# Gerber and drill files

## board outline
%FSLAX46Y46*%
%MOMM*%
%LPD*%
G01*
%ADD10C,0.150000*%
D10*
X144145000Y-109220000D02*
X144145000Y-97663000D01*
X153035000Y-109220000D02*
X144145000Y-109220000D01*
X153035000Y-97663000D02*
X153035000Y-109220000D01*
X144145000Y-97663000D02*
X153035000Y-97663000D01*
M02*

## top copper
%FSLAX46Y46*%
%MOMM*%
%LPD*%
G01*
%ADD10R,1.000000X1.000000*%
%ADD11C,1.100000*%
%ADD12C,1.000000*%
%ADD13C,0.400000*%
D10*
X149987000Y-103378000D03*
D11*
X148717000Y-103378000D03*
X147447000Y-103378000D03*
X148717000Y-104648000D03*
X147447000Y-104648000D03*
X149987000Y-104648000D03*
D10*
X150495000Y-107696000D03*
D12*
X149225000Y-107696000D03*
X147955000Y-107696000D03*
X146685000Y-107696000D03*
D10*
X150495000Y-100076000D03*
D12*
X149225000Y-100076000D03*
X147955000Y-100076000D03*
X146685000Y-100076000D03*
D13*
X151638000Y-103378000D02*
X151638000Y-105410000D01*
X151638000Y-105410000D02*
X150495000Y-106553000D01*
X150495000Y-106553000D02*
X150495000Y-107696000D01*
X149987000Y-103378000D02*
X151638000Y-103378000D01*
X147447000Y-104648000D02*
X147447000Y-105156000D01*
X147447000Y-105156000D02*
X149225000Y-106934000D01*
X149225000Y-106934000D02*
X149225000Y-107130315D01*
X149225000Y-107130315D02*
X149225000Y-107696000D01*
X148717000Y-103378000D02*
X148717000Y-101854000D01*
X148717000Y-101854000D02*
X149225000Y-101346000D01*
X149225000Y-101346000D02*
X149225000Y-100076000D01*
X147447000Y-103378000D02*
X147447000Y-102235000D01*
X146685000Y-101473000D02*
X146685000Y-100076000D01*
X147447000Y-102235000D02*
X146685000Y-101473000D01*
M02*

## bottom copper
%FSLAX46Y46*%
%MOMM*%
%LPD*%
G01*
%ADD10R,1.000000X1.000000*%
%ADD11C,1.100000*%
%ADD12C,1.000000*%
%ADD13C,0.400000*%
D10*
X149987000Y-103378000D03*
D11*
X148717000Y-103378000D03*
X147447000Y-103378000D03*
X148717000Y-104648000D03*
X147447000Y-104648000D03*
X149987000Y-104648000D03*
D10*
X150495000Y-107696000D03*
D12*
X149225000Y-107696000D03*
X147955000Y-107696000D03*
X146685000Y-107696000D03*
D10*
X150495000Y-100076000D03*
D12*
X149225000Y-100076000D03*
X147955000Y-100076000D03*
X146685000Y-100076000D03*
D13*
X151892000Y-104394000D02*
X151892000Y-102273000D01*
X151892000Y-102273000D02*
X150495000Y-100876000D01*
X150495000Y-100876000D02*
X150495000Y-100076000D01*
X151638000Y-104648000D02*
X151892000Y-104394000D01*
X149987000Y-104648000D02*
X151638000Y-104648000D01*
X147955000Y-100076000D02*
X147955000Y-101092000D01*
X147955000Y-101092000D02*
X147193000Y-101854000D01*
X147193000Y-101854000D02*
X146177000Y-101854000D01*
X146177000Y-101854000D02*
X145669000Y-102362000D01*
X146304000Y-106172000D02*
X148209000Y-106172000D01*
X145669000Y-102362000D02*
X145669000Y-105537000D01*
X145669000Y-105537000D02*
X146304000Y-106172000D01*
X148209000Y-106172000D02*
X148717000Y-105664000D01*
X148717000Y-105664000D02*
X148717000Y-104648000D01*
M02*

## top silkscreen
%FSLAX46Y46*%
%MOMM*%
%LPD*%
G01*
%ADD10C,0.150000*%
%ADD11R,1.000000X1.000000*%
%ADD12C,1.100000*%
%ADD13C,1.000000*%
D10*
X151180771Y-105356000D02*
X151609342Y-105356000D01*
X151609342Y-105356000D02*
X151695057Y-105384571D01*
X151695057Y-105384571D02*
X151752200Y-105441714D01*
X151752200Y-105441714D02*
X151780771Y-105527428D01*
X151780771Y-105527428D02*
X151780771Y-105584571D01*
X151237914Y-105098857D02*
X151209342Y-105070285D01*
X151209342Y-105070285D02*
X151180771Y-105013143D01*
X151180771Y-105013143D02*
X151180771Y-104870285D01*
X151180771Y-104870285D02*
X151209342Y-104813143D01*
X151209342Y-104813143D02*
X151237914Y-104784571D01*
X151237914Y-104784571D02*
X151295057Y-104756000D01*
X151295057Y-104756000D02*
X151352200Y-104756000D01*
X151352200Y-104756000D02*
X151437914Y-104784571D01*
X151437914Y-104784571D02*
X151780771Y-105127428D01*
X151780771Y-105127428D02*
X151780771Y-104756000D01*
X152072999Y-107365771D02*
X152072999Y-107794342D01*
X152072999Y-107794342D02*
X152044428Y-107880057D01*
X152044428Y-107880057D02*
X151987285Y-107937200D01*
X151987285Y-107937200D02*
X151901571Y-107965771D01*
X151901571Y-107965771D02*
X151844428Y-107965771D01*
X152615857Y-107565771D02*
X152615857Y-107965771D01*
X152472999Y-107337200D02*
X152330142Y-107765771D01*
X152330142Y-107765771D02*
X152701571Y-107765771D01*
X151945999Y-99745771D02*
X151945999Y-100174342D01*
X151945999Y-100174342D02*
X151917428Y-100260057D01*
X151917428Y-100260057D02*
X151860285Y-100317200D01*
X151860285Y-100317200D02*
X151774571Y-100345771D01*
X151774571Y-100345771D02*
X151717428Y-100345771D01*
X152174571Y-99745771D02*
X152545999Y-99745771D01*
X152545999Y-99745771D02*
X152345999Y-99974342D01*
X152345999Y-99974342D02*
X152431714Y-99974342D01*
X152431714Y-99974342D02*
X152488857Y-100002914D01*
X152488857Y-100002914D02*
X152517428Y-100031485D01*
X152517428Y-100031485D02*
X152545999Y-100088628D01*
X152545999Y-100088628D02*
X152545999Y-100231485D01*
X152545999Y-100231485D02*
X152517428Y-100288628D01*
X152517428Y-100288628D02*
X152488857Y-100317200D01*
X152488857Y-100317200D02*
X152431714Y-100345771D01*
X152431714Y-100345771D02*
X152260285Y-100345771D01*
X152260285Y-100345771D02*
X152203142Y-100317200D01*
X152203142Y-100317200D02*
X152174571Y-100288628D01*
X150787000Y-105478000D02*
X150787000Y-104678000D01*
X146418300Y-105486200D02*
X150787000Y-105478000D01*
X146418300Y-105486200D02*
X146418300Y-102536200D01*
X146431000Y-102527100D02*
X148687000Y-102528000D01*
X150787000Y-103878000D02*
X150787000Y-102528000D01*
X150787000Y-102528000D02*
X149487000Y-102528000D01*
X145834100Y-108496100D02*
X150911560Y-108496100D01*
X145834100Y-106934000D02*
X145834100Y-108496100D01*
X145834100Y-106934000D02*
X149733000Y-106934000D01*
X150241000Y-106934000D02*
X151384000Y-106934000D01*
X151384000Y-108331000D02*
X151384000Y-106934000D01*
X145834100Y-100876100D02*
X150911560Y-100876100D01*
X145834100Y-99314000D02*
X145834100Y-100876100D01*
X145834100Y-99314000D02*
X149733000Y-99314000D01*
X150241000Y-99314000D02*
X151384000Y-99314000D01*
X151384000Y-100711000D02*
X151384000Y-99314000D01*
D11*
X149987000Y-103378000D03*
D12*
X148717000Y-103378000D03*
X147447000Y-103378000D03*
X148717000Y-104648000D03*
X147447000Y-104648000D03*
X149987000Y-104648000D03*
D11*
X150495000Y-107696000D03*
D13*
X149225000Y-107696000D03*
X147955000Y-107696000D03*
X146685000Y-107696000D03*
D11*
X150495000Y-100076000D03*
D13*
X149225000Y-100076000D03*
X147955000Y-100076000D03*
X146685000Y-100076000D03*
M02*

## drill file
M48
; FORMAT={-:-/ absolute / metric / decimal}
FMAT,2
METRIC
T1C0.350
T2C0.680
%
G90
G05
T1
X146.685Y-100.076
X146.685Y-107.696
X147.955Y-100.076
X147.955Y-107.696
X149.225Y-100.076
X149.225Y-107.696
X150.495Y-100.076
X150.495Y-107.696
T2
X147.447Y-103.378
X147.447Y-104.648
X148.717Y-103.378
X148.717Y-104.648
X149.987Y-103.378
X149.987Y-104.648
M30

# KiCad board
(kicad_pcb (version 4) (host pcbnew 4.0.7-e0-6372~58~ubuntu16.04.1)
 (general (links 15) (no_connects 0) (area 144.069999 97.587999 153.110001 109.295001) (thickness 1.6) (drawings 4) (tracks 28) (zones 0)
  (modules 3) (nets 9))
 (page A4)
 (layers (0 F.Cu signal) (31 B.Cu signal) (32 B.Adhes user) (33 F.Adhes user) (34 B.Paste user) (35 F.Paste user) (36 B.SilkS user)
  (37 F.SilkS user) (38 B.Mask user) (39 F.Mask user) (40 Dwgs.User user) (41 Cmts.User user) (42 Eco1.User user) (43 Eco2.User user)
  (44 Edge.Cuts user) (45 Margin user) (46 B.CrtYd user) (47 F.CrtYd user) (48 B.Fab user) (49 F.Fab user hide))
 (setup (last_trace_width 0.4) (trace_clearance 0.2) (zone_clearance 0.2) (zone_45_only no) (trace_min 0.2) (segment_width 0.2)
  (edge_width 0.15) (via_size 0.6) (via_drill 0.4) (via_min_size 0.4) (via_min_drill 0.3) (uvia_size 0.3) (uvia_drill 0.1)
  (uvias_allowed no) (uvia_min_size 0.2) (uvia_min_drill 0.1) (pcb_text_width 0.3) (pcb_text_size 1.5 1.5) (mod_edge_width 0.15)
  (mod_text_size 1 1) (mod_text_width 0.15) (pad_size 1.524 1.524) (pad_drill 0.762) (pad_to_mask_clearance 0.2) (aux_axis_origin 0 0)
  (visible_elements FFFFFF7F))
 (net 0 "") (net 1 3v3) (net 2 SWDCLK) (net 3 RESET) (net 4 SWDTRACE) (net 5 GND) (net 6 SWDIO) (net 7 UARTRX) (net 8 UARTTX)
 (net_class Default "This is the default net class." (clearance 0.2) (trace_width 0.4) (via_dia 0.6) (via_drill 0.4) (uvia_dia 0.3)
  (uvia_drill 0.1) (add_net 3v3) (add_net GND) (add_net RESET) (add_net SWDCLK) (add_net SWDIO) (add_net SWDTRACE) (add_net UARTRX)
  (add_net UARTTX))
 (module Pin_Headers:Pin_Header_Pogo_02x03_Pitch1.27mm (layer F.Cu) (at 149.987 103.378 270)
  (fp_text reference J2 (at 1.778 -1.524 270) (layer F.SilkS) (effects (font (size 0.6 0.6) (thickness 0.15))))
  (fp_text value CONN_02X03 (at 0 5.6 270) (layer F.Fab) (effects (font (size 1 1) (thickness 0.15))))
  (fp_line (start 2.1 -0.8) (end 1.3 -0.8) (layer F.SilkS) (width 0.15))
  (fp_line (start 2.1082 3.5687) (end 2.1 -0.8) (layer F.SilkS) (width 0.15))
  (fp_line (start 2.1082 3.5687) (end -0.8418 3.5687) (layer F.SilkS) (width 0.15))
  (fp_line (start -0.8509 3.556) (end -0.85 1.3) (layer F.SilkS) (width 0.15))
  (fp_line (start 0.5 -0.8) (end -0.85 -0.8) (layer F.SilkS) (width 0.15))
  (fp_line (start -0.85 -0.8) (end -0.85 0.5) (layer F.SilkS) (width 0.15))
  (pad 1 thru_hole rect (at 0 0 270) (size 1 1) (drill 0.68) (layers *.Cu *.Mask F.SilkS) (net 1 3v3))
  (pad 3 thru_hole circle (at 0 1.27 270) (size 1.1 1.1) (drill 0.68) (layers *.Cu *.Mask F.SilkS) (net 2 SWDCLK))
  (pad 5 thru_hole circle (at 0 2.54 270) (size 1.1 1.1) (drill 0.68) (layers *.Cu *.Mask F.SilkS) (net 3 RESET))
  (pad 4 thru_hole circle (at 1.27 1.27 270) (size 1.1 1.1) (drill 0.68) (layers *.Cu *.Mask F.SilkS) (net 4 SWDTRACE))
  (pad 6 thru_hole circle (at 1.27 2.54 270) (size 1.1 1.1) (drill 0.68) (layers *.Cu *.Mask F.SilkS) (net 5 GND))
  (pad 2 thru_hole circle (at 1.27 0 270) (size 1.1 1.1) (drill 0.68) (layers *.Cu *.Mask F.SilkS) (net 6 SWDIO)))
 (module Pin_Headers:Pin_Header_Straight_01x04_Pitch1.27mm (layer F.Cu) (at 150.495 107.696 180)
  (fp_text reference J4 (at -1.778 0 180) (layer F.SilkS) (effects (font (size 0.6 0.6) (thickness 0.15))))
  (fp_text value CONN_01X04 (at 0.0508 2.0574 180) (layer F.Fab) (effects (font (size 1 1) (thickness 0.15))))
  (fp_line (start 4.6609 -0.8001) (end -0.41656 -0.8001) (layer F.SilkS) (width 0.15))
  (fp_line (start 4.6609 0.762) (end 4.6609 -0.8001) (layer F.SilkS) (width 0.15))
  (fp_line (start 4.6609 0.762) (end 0.762 0.762) (layer F.SilkS) (width 0.15))
  (fp_line (start 0.254 0.762) (end -0.889 0.762) (layer F.SilkS) (width 0.15))
  (fp_line (start -0.889 -0.635) (end -0.889 0.762) (layer F.SilkS) (width 0.15))
  (pad 1 thru_hole rect (at 0 0 180) (size 1 1) (drill 0.35) (layers *.Cu *.Mask F.SilkS) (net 1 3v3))
  (pad 2 thru_hole circle (at 1.27 0 180) (size 1 1) (drill 0.35) (layers *.Cu *.Mask F.SilkS) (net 5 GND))
  (pad 3 thru_hole circle (at 2.54 0 180) (size 1 1) (drill 0.35) (layers *.Cu *.Mask F.SilkS) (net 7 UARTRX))
  (pad 4 thru_hole circle (at 3.81 0 180) (size 1 1) (drill 0.35) (layers *.Cu *.Mask F.SilkS) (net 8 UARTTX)))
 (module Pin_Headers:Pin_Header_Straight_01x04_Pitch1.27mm (layer F.Cu) (at 150.495 100.076 180)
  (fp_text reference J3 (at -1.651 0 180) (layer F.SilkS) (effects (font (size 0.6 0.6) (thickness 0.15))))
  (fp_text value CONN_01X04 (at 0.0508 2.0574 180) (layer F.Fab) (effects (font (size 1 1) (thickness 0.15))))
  (fp_line (start 4.6609 -0.8001) (end -0.41656 -0.8001) (layer F.SilkS) (width 0.15))
  (fp_line (start 4.6609 0.762) (end 4.6609 -0.8001) (layer F.SilkS) (width 0.15))
  (fp_line (start 4.6609 0.762) (end 0.762 0.762) (layer F.SilkS) (width 0.15))
  (fp_line (start 0.254 0.762) (end -0.889 0.762) (layer F.SilkS) (width 0.15))
  (fp_line (start -0.889 -0.635) (end -0.889 0.762) (layer F.SilkS) (width 0.15))
  (pad 1 thru_hole rect (at 0 0 180) (size 1 1) (drill 0.35) (layers *.Cu *.Mask F.SilkS) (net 6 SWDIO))
  (pad 2 thru_hole circle (at 1.27 0 180) (size 1 1) (drill 0.35) (layers *.Cu *.Mask F.SilkS) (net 2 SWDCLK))
  (pad 3 thru_hole circle (at 2.54 0 180) (size 1 1) (drill 0.35) (layers *.Cu *.Mask F.SilkS) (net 4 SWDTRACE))
  (pad 4 thru_hole circle (at 3.81 0 180) (size 1 1) (drill 0.35) (layers *.Cu *.Mask F.SilkS) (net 3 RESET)))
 (gr_line (start 144.145 109.22) (end 144.145 97.663) (layer Edge.Cuts) (width 0.15))
 (gr_line (start 153.035 109.22) (end 144.145 109.22) (layer Edge.Cuts) (width 0.15))
 (gr_line (start 153.035 97.663) (end 153.035 109.22) (layer Edge.Cuts) (width 0.15))
 (gr_line (start 144.145 97.663) (end 153.035 97.663) (layer Edge.Cuts) (width 0.15))
 (segment (start 151.638 103.378) (end 151.638 105.41) (width 0.4) (layer F.Cu) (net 1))
 (segment (start 151.638 105.41) (end 150.495 106.553) (width 0.4) (layer F.Cu) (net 1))
 (segment (start 150.495 106.553) (end 150.495 107.696) (width 0.4) (layer F.Cu) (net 1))
 (segment (start 149.987 103.378) (end 151.638 103.378) (width 0.4) (layer F.Cu) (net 1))
 (segment (start 147.447 104.648) (end 147.447 105.156) (width 0.4) (layer F.Cu) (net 5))
 (segment (start 147.447 105.156) (end 149.225 106.934) (width 0.4) (layer F.Cu) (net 5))
 (segment (start 149.225 106.934) (end 149.225 107.130315) (width 0.4) (layer F.Cu) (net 5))
 (segment (start 149.225 107.130315) (end 149.225 107.696) (width 0.4) (layer F.Cu) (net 5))
 (segment (start 148.717 103.378) (end 148.717 101.854) (width 0.4) (layer F.Cu) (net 2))
 (segment (start 148.717 101.854) (end 149.225 101.346) (width 0.4) (layer F.Cu) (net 2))
 (segment (start 149.225 101.346) (end 149.225 100.076) (width 0.4) (layer F.Cu) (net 2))
 (segment (start 147.447 103.378) (end 147.447 102.235) (width 0.4) (layer F.Cu) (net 3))
 (segment (start 146.685 101.473) (end 146.685 100.076) (width 0.4) (layer F.Cu) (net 3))
 (segment (start 147.447 102.235) (end 146.685 101.473) (width 0.4) (layer F.Cu) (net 3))
 (segment (start 151.892 104.394) (end 151.892 102.273) (width 0.4) (layer B.Cu) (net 6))
 (segment (start 151.892 102.273) (end 150.495 100.876) (width 0.4) (layer B.Cu) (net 6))
 (segment (start 150.495 100.876) (end 150.495 100.076) (width 0.4) (layer B.Cu) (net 6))
 (segment (start 151.638 104.648) (end 151.892 104.394) (width 0.4) (layer B.Cu) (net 6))
 (segment (start 149.987 104.648) (end 151.638 104.648) (width 0.4) (layer B.Cu) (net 6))
 (segment (start 147.955 100.076) (end 147.955 101.092) (width 0.4) (layer B.Cu) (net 4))
 (segment (start 147.955 101.092) (end 147.193 101.854) (width 0.4) (layer B.Cu) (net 4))
 (segment (start 147.193 101.854) (end 146.177 101.854) (width 0.4) (layer B.Cu) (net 4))
 (segment (start 146.177 101.854) (end 145.669 102.362) (width 0.4) (layer B.Cu) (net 4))
 (segment (start 146.304 106.172) (end 148.209 106.172) (width 0.4) (layer B.Cu) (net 4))
 (segment (start 145.669 102.362) (end 145.669 105.537) (width 0.4) (layer B.Cu) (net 4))
 (segment (start 145.669 105.537) (end 146.304 106.172) (width 0.4) (layer B.Cu) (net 4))
 (segment (start 148.209 106.172) (end 148.717 105.664) (width 0.4) (layer B.Cu) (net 4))
 (segment (start 148.717 105.664) (end 148.717 104.648) (width 0.4) (layer B.Cu) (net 4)))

